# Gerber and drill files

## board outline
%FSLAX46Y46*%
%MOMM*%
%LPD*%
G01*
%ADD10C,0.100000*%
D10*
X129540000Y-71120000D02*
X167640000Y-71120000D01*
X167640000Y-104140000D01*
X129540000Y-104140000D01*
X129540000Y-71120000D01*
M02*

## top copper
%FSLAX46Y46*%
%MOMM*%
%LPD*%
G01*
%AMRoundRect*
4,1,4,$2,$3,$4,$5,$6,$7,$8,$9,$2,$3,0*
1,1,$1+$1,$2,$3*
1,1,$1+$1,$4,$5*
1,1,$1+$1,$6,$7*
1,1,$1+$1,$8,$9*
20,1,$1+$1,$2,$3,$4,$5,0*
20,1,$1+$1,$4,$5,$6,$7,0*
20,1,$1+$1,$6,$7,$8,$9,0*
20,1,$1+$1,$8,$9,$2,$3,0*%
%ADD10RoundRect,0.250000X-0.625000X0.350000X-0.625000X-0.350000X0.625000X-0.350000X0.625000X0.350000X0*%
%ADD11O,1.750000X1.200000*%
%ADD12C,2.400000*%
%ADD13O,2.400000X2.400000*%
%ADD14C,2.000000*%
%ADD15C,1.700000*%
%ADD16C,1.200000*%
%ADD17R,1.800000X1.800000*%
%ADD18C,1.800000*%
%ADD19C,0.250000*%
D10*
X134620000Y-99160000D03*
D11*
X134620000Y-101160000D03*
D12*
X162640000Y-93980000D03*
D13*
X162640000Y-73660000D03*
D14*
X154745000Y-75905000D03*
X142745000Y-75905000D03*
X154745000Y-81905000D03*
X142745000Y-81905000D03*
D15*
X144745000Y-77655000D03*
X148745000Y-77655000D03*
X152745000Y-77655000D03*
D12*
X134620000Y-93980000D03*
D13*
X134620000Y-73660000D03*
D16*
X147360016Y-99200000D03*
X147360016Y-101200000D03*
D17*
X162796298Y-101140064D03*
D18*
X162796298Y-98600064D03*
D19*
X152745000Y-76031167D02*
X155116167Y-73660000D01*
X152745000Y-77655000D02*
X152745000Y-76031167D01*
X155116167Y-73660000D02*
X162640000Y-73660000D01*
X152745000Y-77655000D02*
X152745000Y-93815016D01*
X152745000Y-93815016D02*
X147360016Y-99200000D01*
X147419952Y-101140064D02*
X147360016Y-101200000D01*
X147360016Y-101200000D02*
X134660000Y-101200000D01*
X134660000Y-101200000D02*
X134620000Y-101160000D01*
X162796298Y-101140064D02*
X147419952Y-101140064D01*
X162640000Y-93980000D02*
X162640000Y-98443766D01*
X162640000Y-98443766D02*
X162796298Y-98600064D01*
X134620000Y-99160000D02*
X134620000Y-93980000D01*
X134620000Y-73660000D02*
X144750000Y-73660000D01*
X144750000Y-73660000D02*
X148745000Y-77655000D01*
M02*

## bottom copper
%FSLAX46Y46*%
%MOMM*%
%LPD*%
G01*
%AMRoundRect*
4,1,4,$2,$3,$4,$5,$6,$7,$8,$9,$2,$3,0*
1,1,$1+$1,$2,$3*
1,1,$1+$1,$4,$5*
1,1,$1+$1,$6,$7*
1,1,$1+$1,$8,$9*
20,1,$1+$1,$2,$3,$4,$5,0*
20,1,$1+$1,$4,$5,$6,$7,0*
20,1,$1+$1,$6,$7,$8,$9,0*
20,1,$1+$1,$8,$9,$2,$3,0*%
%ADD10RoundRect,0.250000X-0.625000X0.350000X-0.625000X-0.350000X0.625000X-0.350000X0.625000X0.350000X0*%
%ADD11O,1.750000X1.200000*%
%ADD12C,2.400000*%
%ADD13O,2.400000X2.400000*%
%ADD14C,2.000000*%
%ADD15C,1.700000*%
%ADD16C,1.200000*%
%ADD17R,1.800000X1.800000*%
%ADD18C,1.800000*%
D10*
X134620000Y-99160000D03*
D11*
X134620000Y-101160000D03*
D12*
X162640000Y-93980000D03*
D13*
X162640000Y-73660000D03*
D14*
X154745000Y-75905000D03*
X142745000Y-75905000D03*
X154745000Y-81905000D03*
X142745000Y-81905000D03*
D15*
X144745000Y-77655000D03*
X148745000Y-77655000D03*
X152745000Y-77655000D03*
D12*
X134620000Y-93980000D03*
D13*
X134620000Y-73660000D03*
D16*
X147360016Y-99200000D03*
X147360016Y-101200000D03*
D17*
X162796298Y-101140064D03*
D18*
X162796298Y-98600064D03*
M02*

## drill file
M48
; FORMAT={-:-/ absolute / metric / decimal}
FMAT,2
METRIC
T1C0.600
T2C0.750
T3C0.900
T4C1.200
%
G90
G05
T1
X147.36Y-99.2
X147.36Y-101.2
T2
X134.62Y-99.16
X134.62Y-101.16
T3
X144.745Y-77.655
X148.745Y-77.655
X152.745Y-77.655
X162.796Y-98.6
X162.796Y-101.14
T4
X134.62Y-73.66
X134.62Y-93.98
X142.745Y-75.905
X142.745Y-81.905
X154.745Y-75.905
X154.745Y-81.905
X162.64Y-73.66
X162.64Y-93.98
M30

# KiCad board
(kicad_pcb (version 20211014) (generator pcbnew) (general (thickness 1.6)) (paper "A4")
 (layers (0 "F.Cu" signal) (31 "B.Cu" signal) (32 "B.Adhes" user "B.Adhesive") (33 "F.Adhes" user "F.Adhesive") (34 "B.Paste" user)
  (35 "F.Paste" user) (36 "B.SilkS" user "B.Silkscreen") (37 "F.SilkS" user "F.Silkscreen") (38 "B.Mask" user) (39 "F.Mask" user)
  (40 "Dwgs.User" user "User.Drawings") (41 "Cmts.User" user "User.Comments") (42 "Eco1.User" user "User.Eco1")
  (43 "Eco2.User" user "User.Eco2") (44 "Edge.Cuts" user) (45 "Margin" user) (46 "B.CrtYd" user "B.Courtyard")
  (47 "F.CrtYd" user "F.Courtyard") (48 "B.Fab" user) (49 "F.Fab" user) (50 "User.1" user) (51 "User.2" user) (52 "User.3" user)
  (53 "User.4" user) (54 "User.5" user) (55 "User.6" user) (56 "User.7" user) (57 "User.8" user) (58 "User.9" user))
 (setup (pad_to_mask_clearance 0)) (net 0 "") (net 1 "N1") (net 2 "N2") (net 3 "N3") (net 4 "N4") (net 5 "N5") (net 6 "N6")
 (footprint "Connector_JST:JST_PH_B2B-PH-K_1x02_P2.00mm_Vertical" (layer "F.Cu") (at 134.62 99.16 -90)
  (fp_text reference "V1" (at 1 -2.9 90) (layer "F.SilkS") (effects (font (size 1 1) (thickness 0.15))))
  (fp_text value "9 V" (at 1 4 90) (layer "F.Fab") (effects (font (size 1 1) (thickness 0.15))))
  (pad "1" thru_hole roundrect (at 0 0 270) (size 1.2 1.75) (drill 0.75) (layers *.Cu *.Mask) (roundrect_rratio 0.208333) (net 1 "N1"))
  (pad "2" thru_hole oval (at 2 0 270) (size 1.2 1.75) (drill 0.75) (layers *.Cu *.Mask) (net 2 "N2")))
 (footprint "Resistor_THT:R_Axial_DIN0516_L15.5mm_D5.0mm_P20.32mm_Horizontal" (layer "F.Cu") (at 162.64 93.98 90)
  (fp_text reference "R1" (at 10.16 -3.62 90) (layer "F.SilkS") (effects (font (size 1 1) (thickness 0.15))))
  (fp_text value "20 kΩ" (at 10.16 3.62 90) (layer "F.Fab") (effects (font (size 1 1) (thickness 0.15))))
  (pad "1" thru_hole circle (at 0 0 90) (size 2.4 2.4) (drill 1.2) (layers *.Cu *.Mask) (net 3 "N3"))
  (pad "2" thru_hole oval (at 20.32 0 90) (size 2.4 2.4) (drill 1.2) (layers *.Cu *.Mask) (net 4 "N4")))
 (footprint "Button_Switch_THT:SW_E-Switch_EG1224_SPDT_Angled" (layer "F.Cu") (at 144.745 77.655)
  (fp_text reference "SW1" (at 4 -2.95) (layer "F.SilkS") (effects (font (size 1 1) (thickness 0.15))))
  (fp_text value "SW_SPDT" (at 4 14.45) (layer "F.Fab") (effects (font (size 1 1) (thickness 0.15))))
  (pad "" thru_hole circle (at 10 -1.75) (size 2 2) (drill 1.2) (layers *.Cu *.Mask))
  (pad "" thru_hole circle (at -2 -1.75) (size 2 2) (drill 1.2) (layers *.Cu *.Mask))
  (pad "" thru_hole circle (at 10 4.25) (size 2 2) (drill 1.2) (layers *.Cu *.Mask))
  (pad "" thru_hole circle (at -2 4.25) (size 2 2) (drill 1.2) (layers *.Cu *.Mask))
  (pad "1" thru_hole circle (at 0 0) (size 1.7 1.7) (drill 0.9) (layers *.Cu *.Mask) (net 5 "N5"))
  (pad "2" thru_hole circle (at 4 0) (size 1.7 1.7) (drill 0.9) (layers *.Cu *.Mask) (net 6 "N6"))
  (pad "3" thru_hole circle (at 8 0) (size 1.7 1.7) (drill 0.9) (layers *.Cu *.Mask) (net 4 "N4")))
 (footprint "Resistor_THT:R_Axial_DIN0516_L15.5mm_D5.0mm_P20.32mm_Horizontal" (layer "F.Cu") (at 134.62 93.98 90)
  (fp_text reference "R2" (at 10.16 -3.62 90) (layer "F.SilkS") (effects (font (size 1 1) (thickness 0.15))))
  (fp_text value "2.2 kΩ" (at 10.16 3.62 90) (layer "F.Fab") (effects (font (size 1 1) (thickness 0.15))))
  (pad "1" thru_hole circle (at 0 0 90) (size 2.4 2.4) (drill 1.2) (layers *.Cu *.Mask) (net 1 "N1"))
  (pad "2" thru_hole oval (at 20.32 0 90) (size 2.4 2.4) (drill 1.2) (layers *.Cu *.Mask) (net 6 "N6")))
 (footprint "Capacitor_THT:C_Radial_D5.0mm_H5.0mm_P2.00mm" (layer "F.Cu") (at 147.360016 99.2 -90)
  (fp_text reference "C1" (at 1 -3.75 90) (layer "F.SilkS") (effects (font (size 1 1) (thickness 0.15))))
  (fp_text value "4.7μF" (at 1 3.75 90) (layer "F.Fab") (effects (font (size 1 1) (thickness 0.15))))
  (pad "1" thru_hole circle (at 0 0 270) (size 1.2 1.2) (drill 0.6) (layers *.Cu *.Mask) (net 4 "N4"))
  (pad "2" thru_hole circle (at 2 0 270) (size 1.2 1.2) (drill 0.6) (layers *.Cu *.Mask) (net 2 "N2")))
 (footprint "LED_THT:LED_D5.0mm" (layer "F.Cu") (at 162.796298 101.140064 90)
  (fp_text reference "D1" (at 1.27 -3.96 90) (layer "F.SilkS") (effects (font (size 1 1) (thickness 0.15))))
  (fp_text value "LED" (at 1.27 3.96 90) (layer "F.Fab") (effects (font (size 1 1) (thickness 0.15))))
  (pad "1" thru_hole rect (at 0 0 90) (size 1.8 1.8) (drill 0.9) (layers *.Cu *.Mask) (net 2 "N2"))
  (pad "2" thru_hole circle (at 2.54 0 90) (size 1.8 1.8) (drill 0.9) (layers *.Cu *.Mask) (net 3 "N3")))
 (gr_rect (start 129.54 71.12) (end 167.64 104.14) (layer "Edge.Cuts") (width 0.1) (fill none))
 (segment (start 152.745 76.031167) (end 155.116167 73.66) (width 0.25) (layer "F.Cu") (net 4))
 (segment (start 152.745 77.655) (end 152.745 76.031167) (width 0.25) (layer "F.Cu") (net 4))
 (segment (start 155.116167 73.66) (end 162.64 73.66) (width 0.25) (layer "F.Cu") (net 4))
 (segment (start 152.745 77.655) (end 152.745 93.815016) (width 0.25) (layer "F.Cu") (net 4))
 (segment (start 152.745 93.815016) (end 147.360016 99.2) (width 0.25) (layer "F.Cu") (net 4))
 (segment (start 147.419952 101.140064) (end 147.360016 101.2) (width 0.25) (layer "F.Cu") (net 2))
 (segment (start 147.360016 101.2) (end 134.66 101.2) (width 0.25) (layer "F.Cu") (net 2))
 (segment (start 134.66 101.2) (end 134.62 101.16) (width 0.25) (layer "F.Cu") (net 2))
 (segment (start 162.796298 101.140064) (end 147.419952 101.140064) (width 0.25) (layer "F.Cu") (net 2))
 (segment (start 162.64 93.98) (end 162.64 98.443766) (width 0.25) (layer "F.Cu") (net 3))
 (segment (start 162.64 98.443766) (end 162.796298 98.600064) (width 0.25) (layer "F.Cu") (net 3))
 (segment (start 134.62 99.16) (end 134.62 93.98) (width 0.25) (layer "F.Cu") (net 1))
 (segment (start 134.62 73.66) (end 144.75 73.66) (width 0.25) (layer "F.Cu") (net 6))
 (segment (start 144.75 73.66) (end 148.745 77.655) (width 0.25) (layer "F.Cu") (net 6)))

